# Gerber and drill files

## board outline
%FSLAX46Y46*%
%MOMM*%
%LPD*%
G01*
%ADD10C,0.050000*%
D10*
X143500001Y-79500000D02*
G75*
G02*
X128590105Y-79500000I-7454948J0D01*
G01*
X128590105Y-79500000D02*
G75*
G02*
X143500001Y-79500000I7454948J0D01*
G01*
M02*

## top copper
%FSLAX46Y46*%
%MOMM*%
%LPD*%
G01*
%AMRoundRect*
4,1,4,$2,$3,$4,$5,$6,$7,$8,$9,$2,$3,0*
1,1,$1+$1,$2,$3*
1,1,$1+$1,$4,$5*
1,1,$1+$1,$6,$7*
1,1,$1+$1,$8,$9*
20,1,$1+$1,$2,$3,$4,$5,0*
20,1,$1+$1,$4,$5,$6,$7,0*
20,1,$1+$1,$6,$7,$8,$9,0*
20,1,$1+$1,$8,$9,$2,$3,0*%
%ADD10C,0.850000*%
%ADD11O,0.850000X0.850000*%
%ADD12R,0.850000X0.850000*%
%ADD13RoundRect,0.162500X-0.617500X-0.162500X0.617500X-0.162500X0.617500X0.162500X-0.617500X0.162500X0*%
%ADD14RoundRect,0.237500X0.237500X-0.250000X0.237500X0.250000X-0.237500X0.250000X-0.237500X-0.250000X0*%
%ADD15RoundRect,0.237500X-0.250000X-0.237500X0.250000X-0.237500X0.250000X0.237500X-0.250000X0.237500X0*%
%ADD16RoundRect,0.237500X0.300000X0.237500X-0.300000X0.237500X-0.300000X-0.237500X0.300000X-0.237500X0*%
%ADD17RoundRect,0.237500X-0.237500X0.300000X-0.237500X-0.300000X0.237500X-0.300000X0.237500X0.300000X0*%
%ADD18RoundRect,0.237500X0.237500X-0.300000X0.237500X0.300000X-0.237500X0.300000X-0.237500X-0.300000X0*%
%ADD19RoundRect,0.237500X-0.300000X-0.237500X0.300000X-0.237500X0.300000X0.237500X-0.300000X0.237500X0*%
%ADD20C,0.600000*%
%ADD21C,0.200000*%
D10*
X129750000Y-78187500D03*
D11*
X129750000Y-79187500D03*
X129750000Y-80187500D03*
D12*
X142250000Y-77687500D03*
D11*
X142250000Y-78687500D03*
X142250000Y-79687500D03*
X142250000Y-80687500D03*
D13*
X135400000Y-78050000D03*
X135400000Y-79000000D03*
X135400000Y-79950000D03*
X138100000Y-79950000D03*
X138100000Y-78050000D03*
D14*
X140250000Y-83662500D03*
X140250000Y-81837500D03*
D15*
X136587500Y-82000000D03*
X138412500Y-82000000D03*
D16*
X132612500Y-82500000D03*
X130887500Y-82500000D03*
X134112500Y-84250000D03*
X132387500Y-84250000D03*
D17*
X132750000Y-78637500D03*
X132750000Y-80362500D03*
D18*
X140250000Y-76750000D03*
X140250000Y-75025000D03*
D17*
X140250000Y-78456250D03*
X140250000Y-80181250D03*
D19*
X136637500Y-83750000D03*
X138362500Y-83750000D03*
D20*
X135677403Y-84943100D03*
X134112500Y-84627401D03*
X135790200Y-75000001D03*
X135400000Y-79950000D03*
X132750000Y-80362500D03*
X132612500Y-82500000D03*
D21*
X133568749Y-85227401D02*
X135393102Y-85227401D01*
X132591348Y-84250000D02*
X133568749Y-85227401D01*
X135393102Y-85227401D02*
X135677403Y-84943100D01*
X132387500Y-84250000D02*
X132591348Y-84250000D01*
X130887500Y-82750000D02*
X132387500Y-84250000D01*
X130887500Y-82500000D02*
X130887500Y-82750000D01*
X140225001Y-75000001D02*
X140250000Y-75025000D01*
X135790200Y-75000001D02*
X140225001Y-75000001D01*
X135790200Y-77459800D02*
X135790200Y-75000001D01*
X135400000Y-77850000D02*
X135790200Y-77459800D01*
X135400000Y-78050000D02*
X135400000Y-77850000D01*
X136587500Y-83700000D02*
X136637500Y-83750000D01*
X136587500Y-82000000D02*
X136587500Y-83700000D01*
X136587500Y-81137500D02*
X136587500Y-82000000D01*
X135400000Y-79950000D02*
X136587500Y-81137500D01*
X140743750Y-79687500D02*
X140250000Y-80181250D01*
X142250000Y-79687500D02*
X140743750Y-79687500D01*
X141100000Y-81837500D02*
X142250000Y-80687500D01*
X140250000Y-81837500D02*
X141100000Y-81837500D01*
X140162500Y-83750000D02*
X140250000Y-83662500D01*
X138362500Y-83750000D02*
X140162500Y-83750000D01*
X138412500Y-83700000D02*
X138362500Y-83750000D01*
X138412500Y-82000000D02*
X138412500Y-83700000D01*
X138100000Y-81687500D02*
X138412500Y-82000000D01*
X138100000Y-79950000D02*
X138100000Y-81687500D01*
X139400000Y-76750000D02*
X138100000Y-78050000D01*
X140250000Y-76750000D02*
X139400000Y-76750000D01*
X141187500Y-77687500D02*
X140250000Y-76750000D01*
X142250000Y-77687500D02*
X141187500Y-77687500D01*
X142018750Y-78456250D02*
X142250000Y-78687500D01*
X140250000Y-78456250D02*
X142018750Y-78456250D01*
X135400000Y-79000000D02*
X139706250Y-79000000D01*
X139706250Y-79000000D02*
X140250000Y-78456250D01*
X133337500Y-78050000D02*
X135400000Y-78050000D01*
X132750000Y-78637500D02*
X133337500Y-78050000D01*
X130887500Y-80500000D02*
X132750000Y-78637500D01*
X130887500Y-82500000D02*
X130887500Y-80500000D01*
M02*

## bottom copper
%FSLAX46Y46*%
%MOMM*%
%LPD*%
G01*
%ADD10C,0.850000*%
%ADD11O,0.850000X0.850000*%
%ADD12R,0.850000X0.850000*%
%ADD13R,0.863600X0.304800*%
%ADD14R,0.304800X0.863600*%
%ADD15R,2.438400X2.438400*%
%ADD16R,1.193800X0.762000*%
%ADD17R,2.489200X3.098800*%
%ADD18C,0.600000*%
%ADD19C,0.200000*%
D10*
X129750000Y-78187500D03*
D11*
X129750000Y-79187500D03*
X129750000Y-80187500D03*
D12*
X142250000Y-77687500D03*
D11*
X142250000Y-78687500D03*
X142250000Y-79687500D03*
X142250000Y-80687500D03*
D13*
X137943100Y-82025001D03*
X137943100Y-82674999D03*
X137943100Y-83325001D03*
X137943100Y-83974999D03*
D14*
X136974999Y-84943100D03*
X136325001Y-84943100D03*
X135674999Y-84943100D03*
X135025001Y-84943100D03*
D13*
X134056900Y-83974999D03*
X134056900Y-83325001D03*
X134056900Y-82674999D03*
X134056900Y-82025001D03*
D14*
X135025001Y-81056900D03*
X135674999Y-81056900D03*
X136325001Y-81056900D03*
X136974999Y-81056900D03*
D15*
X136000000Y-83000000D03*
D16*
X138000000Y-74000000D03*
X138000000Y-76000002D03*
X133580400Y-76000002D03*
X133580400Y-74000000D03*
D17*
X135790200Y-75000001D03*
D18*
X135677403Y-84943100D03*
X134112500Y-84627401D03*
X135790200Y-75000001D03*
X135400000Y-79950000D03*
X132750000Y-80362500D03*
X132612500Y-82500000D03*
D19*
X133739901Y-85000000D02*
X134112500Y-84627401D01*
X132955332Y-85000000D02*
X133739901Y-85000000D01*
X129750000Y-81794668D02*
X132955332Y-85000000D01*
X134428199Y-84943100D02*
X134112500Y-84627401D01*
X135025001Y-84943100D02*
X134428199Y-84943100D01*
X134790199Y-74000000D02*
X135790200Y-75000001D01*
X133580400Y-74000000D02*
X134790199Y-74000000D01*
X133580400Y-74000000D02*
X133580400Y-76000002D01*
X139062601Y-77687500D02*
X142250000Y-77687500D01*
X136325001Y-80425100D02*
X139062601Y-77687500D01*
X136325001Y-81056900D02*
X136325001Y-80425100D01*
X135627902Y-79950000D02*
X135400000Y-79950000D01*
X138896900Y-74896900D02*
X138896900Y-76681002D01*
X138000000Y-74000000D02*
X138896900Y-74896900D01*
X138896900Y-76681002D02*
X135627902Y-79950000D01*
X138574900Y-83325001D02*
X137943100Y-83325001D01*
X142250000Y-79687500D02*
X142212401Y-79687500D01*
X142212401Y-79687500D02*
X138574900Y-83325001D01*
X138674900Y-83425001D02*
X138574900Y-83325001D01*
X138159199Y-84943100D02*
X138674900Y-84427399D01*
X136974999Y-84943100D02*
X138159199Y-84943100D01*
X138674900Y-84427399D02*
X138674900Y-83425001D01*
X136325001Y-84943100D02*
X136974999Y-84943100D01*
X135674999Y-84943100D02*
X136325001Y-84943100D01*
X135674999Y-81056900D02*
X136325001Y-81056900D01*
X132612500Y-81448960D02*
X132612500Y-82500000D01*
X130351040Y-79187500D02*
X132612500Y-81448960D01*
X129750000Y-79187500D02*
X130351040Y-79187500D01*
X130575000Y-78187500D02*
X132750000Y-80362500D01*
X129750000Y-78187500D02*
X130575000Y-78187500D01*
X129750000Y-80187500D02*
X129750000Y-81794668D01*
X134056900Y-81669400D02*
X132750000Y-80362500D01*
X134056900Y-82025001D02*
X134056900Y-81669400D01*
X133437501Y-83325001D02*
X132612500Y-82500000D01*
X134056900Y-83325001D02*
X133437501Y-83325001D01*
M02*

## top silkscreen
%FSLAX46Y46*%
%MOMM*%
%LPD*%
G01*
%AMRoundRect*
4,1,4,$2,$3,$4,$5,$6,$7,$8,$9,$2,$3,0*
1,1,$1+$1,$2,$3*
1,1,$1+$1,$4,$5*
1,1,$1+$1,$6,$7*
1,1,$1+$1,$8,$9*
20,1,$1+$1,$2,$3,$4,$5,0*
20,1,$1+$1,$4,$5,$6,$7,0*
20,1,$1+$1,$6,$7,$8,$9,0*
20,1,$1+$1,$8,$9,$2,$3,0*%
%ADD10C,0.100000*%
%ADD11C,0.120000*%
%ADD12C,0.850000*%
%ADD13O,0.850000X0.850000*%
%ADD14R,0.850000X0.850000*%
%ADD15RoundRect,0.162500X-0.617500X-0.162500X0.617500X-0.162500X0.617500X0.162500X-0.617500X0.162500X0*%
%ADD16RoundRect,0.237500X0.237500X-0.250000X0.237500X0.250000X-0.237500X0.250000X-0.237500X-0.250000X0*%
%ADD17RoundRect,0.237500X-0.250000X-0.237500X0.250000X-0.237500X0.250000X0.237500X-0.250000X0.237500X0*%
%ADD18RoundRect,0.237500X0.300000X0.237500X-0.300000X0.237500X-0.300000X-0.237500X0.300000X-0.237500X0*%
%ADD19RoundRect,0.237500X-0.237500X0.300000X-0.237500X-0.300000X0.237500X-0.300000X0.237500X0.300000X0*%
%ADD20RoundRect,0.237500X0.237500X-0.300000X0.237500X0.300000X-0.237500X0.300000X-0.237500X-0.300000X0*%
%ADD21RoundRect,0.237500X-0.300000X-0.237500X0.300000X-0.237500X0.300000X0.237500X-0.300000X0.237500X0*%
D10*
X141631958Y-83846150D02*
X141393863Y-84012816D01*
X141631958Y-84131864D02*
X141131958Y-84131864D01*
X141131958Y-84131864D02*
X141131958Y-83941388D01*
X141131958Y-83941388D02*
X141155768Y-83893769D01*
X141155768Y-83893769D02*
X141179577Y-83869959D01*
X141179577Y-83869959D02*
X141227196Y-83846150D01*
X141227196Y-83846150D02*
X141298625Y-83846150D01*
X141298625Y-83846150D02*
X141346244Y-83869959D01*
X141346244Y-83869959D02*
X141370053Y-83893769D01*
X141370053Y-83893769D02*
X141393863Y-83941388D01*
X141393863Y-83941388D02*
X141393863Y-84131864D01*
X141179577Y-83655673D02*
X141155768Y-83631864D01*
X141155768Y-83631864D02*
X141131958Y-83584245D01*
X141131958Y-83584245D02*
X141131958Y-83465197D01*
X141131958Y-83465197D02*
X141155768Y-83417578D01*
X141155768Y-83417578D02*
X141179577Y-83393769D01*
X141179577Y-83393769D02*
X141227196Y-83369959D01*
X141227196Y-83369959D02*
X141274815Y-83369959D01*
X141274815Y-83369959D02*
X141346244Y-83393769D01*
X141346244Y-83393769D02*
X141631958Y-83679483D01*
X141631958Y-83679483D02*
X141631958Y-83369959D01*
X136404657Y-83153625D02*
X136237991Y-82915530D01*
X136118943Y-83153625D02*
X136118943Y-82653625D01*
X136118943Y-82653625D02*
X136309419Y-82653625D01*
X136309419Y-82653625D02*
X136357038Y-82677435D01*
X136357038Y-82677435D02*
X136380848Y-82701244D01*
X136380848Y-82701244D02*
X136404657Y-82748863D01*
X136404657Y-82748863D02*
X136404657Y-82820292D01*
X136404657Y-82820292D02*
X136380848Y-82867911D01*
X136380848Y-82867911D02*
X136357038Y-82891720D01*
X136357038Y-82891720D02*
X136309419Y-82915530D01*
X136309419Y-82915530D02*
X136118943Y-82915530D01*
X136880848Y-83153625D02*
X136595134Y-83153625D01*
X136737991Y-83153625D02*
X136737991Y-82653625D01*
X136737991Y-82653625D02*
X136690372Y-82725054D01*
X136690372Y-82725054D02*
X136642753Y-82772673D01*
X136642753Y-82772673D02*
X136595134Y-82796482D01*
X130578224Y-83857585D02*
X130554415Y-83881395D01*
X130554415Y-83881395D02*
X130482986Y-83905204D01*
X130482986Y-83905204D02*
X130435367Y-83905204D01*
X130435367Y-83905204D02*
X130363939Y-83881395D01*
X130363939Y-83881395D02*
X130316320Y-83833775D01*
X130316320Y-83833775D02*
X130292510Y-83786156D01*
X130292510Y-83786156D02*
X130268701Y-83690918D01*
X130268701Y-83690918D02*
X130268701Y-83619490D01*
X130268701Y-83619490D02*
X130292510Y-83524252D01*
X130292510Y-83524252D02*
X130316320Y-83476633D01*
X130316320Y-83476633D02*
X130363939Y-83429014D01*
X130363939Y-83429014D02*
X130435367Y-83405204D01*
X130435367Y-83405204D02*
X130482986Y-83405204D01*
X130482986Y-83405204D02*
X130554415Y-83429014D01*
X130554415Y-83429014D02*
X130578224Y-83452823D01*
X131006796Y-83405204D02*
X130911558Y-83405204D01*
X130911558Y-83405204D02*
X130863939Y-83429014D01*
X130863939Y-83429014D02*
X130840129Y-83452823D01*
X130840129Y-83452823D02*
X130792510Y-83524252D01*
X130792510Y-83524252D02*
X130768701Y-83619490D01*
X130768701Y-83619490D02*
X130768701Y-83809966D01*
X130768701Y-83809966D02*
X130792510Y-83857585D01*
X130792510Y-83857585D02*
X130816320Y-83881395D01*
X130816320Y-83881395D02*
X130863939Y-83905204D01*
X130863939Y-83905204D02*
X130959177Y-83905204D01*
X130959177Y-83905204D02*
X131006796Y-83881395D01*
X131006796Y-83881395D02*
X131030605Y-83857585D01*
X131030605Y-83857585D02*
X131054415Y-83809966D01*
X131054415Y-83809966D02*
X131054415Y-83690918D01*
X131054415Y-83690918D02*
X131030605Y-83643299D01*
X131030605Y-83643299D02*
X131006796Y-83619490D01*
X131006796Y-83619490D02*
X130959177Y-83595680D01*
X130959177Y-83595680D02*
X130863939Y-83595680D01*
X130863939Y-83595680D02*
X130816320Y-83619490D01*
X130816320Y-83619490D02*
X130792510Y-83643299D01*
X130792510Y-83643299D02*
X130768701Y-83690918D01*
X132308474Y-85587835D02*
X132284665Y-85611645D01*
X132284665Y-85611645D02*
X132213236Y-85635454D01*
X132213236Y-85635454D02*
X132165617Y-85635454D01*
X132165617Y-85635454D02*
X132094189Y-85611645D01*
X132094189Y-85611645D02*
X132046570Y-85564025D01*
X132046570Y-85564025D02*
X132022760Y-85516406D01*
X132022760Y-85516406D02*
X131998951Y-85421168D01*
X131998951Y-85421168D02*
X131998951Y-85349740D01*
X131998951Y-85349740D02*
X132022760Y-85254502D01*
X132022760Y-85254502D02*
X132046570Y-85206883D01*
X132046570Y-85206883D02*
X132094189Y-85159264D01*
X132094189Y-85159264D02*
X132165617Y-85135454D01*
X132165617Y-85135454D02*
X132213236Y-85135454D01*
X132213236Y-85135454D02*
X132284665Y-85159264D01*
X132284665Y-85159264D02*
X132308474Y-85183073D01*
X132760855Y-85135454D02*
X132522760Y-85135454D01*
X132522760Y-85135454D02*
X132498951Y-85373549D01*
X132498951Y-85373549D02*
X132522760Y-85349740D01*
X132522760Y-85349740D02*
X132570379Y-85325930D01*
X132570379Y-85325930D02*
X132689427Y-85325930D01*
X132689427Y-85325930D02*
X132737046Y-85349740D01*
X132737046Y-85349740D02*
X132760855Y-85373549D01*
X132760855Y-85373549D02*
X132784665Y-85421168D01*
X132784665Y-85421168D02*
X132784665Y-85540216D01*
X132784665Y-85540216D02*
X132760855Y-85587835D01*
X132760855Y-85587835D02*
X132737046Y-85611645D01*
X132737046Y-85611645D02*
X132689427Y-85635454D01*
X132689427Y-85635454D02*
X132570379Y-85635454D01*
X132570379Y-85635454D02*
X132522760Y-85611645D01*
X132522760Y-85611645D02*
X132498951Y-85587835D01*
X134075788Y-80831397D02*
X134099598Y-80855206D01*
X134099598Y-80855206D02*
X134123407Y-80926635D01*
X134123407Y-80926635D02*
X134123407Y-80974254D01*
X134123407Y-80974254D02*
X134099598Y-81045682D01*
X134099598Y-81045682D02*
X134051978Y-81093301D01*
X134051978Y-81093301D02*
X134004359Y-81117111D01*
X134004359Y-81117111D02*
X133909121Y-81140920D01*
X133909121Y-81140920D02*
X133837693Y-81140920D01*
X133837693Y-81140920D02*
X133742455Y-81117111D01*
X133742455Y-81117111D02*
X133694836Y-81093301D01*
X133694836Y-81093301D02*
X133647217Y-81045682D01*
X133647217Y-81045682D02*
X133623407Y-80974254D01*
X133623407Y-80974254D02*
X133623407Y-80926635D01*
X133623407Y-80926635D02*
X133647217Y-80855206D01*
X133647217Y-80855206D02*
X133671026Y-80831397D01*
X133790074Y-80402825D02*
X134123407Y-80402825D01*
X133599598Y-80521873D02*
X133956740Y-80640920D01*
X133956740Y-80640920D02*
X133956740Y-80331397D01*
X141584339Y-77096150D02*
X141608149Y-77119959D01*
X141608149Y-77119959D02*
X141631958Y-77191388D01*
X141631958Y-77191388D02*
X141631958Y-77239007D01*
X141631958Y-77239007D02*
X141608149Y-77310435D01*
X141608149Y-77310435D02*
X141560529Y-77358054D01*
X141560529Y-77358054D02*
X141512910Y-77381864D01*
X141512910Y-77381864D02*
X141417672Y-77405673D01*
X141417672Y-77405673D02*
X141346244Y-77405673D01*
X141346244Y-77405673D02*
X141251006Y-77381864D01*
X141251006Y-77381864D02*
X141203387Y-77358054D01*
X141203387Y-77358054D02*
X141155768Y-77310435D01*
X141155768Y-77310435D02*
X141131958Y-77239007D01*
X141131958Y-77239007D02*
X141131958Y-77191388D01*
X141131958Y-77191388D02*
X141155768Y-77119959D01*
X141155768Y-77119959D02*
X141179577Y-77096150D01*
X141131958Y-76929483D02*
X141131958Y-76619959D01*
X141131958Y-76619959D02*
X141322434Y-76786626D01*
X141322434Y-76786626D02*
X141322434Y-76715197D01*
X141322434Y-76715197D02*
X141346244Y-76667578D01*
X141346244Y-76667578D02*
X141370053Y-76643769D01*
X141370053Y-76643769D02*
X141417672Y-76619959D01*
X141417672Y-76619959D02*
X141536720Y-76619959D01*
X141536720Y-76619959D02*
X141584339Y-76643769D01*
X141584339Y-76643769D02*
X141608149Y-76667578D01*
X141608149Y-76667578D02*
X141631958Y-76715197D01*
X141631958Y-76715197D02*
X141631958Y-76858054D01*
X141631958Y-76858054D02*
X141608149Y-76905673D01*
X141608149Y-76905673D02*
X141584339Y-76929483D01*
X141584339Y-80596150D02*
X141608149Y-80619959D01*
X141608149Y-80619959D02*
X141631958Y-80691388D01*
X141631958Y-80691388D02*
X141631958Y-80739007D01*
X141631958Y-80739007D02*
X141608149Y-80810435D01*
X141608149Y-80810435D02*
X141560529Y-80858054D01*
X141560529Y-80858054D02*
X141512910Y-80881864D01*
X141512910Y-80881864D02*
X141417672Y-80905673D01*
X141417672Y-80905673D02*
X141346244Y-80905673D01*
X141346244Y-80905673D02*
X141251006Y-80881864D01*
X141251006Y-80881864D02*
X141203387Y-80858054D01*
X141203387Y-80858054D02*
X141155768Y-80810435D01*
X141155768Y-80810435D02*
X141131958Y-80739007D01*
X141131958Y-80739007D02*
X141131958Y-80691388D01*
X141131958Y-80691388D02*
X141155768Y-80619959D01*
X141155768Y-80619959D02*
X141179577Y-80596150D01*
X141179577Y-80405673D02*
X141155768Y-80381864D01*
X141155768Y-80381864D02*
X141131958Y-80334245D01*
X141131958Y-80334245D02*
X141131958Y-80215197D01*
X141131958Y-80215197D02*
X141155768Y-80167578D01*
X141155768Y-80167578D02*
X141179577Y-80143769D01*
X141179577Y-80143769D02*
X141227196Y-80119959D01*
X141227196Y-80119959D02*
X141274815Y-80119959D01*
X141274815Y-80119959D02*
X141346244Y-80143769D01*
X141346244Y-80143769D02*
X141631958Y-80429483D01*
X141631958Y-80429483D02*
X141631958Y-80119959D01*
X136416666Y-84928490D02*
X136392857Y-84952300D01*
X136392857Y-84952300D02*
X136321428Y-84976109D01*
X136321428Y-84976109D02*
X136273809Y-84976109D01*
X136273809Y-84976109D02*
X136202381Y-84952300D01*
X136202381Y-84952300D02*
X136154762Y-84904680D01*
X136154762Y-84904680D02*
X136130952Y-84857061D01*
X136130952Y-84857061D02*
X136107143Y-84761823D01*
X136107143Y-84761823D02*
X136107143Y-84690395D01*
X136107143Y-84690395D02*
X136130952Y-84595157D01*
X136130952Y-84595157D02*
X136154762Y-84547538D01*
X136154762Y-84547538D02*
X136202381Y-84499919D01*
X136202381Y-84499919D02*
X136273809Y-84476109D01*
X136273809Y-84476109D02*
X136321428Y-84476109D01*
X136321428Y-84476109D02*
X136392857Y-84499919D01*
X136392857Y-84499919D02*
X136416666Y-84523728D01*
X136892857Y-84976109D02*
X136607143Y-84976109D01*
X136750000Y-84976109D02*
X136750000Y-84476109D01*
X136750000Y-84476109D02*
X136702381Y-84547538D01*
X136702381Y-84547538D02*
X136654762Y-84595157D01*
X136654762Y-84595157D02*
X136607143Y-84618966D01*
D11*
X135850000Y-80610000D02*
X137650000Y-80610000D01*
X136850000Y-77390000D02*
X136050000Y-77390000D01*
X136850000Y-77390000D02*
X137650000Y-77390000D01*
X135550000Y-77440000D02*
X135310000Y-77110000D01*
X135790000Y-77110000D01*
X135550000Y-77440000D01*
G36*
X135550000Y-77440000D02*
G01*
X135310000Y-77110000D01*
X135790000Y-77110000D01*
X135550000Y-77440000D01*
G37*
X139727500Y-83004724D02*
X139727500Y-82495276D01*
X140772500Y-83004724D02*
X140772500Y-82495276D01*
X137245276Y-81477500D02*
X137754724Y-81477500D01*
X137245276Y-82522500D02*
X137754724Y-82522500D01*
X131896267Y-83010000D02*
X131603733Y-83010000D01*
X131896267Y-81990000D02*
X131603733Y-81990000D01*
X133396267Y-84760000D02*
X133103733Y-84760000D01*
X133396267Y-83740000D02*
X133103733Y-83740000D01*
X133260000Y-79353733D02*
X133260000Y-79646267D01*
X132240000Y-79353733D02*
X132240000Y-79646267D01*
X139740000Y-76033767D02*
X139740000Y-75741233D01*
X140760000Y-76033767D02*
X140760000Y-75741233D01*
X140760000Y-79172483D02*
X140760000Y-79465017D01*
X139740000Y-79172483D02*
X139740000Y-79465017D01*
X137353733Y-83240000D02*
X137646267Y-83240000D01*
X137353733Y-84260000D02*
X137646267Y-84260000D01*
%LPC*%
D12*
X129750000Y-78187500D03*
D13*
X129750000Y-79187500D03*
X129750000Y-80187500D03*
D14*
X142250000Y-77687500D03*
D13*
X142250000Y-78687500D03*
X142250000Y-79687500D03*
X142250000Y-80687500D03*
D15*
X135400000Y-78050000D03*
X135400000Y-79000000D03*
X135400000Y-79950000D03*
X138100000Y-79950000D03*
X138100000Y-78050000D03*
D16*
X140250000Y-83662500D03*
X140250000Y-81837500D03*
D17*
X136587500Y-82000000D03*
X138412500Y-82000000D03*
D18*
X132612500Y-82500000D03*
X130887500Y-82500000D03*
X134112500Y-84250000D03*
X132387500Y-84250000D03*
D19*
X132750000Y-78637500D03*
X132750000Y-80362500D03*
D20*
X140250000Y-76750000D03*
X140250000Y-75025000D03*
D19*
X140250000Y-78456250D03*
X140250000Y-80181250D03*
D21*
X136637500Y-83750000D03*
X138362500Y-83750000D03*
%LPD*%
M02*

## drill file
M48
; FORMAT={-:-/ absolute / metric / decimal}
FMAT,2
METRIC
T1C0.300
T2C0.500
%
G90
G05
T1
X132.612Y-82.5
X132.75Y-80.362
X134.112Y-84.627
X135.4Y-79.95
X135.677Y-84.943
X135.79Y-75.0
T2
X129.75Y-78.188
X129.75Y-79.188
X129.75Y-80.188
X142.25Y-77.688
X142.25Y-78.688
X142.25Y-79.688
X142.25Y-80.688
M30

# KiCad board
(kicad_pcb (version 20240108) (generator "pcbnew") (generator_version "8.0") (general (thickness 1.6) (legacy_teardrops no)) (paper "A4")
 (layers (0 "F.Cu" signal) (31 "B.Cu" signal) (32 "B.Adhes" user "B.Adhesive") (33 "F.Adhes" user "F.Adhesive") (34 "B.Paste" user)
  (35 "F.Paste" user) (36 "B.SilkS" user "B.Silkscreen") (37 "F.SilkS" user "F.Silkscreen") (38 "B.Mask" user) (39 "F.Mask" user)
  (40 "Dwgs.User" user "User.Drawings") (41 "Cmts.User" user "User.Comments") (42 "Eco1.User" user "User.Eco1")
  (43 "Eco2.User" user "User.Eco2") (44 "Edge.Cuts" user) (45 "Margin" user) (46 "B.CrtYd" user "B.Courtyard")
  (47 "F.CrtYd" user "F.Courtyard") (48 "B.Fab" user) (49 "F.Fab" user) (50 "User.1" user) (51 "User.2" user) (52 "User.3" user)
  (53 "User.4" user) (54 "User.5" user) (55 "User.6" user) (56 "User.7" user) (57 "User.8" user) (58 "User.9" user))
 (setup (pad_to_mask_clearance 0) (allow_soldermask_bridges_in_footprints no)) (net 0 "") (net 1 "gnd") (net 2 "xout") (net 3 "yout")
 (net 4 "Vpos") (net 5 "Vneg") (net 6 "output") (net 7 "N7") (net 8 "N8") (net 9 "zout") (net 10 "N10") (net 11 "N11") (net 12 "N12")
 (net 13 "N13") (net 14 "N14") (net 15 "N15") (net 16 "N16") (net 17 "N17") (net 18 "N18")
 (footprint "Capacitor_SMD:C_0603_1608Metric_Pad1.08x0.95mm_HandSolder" (layer "F.Cu") (at 132.75 79.5 -90)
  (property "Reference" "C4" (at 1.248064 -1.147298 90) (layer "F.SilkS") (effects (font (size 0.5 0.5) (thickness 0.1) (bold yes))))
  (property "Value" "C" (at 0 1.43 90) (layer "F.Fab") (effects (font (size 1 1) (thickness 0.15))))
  (fp_line (start -0.146267 0.51) (end 0.146267 0.51) (stroke (width 0.12) (type solid)) (layer "F.SilkS"))
  (fp_line (start -0.146267 -0.51) (end 0.146267 -0.51) (stroke (width 0.12) (type solid)) (layer "F.SilkS"))
  (pad "1" smd roundrect (at -0.8625 0 270) (size 1.075 0.95) (layers "F.Cu" "F.Paste" "F.Mask") (roundrect_rratio 0.25) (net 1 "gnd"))
  (pad "2" smd roundrect (at 0.8625 0 270) (size 1.075 0.95) (layers "F.Cu" "F.Paste" "F.Mask") (roundrect_rratio 0.25) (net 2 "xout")))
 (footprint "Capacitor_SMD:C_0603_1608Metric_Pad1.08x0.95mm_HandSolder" (layer "F.Cu") (at 131.75 82.5 180)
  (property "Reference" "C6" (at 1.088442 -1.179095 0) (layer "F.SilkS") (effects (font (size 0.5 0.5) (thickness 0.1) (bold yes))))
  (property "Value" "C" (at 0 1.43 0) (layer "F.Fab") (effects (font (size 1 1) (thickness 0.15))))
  (fp_line (start -0.146267 0.51) (end 0.146267 0.51) (stroke (width 0.12) (type solid)) (layer "F.SilkS"))
  (fp_line (start -0.146267 -0.51) (end 0.146267 -0.51) (stroke (width 0.12) (type solid)) (layer "F.SilkS"))
  (pad "1" smd roundrect (at -0.8625 0 180) (size 1.075 0.95) (layers "F.Cu" "F.Paste" "F.Mask") (roundrect_rratio 0.25) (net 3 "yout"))
  (pad "2" smd roundrect (at 0.8625 0 180) (size 1.075 0.95) (layers "F.Cu" "F.Paste" "F.Mask") (roundrect_rratio 0.25) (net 1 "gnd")))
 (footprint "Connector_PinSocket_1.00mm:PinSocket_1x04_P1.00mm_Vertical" (layer "F.Cu") (at 142.25 77.6875)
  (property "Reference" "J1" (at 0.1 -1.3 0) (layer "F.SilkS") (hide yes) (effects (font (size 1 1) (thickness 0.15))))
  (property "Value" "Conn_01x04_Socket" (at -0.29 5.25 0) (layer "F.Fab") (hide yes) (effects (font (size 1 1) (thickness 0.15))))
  (pad "1" thru_hole rect (at 0 0) (size 0.85 0.85) (drill 0.5) (layers "*.Cu" "*.Mask") (remove_unused_layers no) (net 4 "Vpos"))
  (pad "2" thru_hole oval (at 0 1) (size 0.85 0.85) (drill 0.5) (layers "*.Cu" "*.Mask") (remove_unused_layers no) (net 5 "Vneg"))
  (pad "3" thru_hole oval (at 0 2) (size 0.85 0.85) (drill 0.5) (layers "*.Cu" "*.Mask") (remove_unused_layers no) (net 1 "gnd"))
  (pad "4" thru_hole oval (at 0 3) (size 0.85 0.85) (drill 0.5) (layers "*.Cu" "*.Mask") (remove_unused_layers no) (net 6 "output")))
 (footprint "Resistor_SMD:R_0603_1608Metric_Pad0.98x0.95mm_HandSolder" (layer "F.Cu") (at 137.5 82)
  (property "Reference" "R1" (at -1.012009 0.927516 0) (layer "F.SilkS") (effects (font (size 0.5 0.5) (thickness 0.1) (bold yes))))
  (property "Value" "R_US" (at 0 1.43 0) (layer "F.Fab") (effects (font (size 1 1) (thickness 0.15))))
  (fp_line (start -0.254724 -0.5225) (end 0.254724 -0.5225) (stroke (width 0.12) (type solid)) (layer "F.SilkS"))
  (fp_line (start -0.254724 0.5225) (end 0.254724 0.5225) (stroke (width 0.12) (type solid)) (layer "F.SilkS"))
  (pad "1" smd roundrect (at -0.9125 0) (size 0.975 0.95) (layers "F.Cu" "F.Paste" "F.Mask") (roundrect_rratio 0.25) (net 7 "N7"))
  (pad "2" smd roundrect (at 0.9125 0) (size 0.975 0.95) (layers "F.Cu" "F.Paste" "F.Mask") (roundrect_rratio 0.25) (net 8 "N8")))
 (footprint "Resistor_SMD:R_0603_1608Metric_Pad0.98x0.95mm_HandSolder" (layer "F.Cu") (at 140.25 82.75 90)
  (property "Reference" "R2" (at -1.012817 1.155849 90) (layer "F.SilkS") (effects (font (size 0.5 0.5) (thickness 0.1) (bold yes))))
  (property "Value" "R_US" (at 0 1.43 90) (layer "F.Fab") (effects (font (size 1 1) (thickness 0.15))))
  (fp_line (start -0.254724 -0.5225) (end 0.254724 -0.5225) (stroke (width 0.12) (type solid)) (layer "F.SilkS"))
  (fp_line (start -0.254724 0.5225) (end 0.254724 0.5225) (stroke (width 0.12) (type solid)) (layer "F.SilkS"))
  (pad "1" smd roundrect (at -0.9125 0 90) (size 0.975 0.95) (layers "F.Cu" "F.Paste" "F.Mask") (roundrect_rratio 0.25) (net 8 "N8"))
  (pad "2" smd roundrect (at 0.9125 0 90) (size 0.975 0.95) (layers "F.Cu" "F.Paste" "F.Mask") (roundrect_rratio 0.25) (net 6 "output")))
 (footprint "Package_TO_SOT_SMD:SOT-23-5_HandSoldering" (layer "F.Cu") (at 136.75 79)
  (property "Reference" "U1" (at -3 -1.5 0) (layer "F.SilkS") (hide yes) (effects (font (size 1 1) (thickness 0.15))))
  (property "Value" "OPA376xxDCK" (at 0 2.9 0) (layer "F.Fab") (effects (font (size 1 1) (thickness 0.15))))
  (fp_line (start -0.9 1.61) (end 0.9 1.61) (stroke (width 0.12) (type solid)) (layer "F.SilkS"))
  (fp_line (start 0.1 -1.61) (end -0.7 -1.61) (stroke (width 0.12) (type solid)) (layer "F.SilkS"))
  (fp_line (start 0.1 -1.61) (end 0.9 -1.61) (stroke (width 0.12) (type solid)) (layer "F.SilkS"))
  (fp_poly
   (pts (xy -1.2 -1.56) (xy -1.44 -1.89) (xy -0.96 -1.89) (xy -1.2 -1.56)) (stroke (width 0.12) (type solid)) (fill solid) (layer "F.SilkS"))
  (pad "1" smd roundrect (at -1.35 -0.95) (size 1.56 0.65) (layers "F.Cu" "F.Paste" "F.Mask") (roundrect_rratio 0.25) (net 1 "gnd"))
  (pad "2" smd roundrect (at -1.35 0) (size 1.56 0.65) (layers "F.Cu" "F.Paste" "F.Mask") (roundrect_rratio 0.25) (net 5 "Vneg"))
  (pad "3" smd roundrect (at -1.35 0.95) (size 1.56 0.65) (layers "F.Cu" "F.Paste" "F.Mask") (roundrect_rratio 0.25) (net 7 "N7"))
  (pad "4" smd roundrect (at 1.35 0.95) (size 1.56 0.65) (layers "F.Cu" "F.Paste" "F.Mask") (roundrect_rratio 0.25) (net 8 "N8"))
  (pad "5" smd roundrect (at 1.35 -0.95) (size 1.56 0.65) (layers "F.Cu" "F.Paste" "F.Mask") (roundrect_rratio 0.25) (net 4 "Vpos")))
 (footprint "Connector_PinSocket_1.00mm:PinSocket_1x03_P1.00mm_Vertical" (layer "F.Cu") (at 129.75 78.1875)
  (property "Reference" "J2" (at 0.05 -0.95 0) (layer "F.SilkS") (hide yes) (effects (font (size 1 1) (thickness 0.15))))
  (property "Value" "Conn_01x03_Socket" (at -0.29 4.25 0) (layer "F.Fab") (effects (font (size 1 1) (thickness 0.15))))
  (pad "1" thru_hole circle (at 0 0) (size 0.85 0.85) (drill 0.5) (layers "*.Cu" "*.Mask") (remove_unused_layers no) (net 2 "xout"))
  (pad "2" thru_hole oval (at 0 1) (size 0.85 0.85) (drill 0.5) (layers "*.Cu" "*.Mask") (remove_unused_layers no) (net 3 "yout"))
  (pad "3" thru_hole oval (at 0 2) (size 0.85 0.85) (drill 0.5) (layers "*.Cu" "*.Mask") (remove_unused_layers no) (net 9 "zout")))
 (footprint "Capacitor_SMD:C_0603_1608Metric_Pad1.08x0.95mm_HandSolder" (layer "F.Cu") (at 140.25 79.31875 -90)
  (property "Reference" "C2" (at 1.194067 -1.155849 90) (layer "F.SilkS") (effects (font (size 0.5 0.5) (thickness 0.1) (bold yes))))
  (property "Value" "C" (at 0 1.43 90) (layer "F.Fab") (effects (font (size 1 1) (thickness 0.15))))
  (fp_line (start -0.146267 0.51) (end 0.146267 0.51) (stroke (width 0.12) (type solid)) (layer "F.SilkS"))
  (fp_line (start -0.146267 -0.51) (end 0.146267 -0.51) (stroke (width 0.12) (type solid)) (layer "F.SilkS"))
  (pad "1" smd roundrect (at -0.8625 0 270) (size 1.075 0.95) (layers "F.Cu" "F.Paste" "F.Mask") (roundrect_rratio 0.25) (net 5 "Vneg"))
  (pad "2" smd roundrect (at 0.8625 0 270) (size 1.075 0.95) (layers "F.Cu" "F.Paste" "F.Mask") (roundrect_rratio 0.25) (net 1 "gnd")))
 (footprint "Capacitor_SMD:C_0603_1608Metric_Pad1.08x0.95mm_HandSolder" (layer "F.Cu") (at 140.25 75.8875 90)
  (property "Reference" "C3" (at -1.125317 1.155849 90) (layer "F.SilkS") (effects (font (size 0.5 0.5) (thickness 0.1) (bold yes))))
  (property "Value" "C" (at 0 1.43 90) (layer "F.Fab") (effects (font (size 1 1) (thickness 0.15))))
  (fp_line (start -0.146267 -0.51) (end 0.146267 -0.51) (stroke (width 0.12) (type solid)) (layer "F.SilkS"))
  (fp_line (start -0.146267 0.51) (end 0.146267 0.51) (stroke (width 0.12) (type solid)) (layer "F.SilkS"))
  (pad "1" smd roundrect (at -0.8625 0 90) (size 1.075 0.95) (layers "F.Cu" "F.Paste" "F.Mask") (roundrect_rratio 0.25) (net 4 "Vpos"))
  (pad "2" smd roundrect (at 0.8625 0 90) (size 1.075 0.95) (layers "F.Cu" "F.Paste" "F.Mask") (roundrect_rratio 0.25) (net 1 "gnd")))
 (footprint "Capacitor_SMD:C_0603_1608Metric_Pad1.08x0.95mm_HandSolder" (layer "F.Cu") (at 133.25 84.25 180)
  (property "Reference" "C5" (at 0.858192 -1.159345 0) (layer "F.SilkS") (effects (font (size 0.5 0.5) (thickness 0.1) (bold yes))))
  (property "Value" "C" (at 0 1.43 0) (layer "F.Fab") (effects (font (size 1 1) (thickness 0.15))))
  (fp_line (start -0.146267 0.51) (end 0.146267 0.51) (stroke (width 0.12) (type solid)) (layer "F.SilkS"))
  (fp_line (start -0.146267 -0.51) (end 0.146267 -0.51) (stroke (width 0.12) (type solid)) (layer "F.SilkS"))
  (pad "1" smd roundrect (at -0.8625 0 180) (size 1.075 0.95) (layers "F.Cu" "F.Paste" "F.Mask") (roundrect_rratio 0.25) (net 9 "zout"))
  (pad "2" smd roundrect (at 0.8625 0 180) (size 1.075 0.95) (layers "F.Cu" "F.Paste" "F.Mask") (roundrect_rratio 0.25) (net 1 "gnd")))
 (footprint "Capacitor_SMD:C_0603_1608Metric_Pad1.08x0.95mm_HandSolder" (layer "F.Cu") (at 137.5 83.75)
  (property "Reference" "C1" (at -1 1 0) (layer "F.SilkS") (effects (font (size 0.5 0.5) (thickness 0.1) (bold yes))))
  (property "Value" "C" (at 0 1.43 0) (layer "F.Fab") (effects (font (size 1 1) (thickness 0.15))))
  (fp_line (start -0.146267 -0.51) (end 0.146267 -0.51) (stroke (width 0.12) (type solid)) (layer "F.SilkS"))
  (fp_line (start -0.146267 0.51) (end 0.146267 0.51) (stroke (width 0.12) (type solid)) (layer "F.SilkS"))
  (pad "1" smd roundrect (at -0.8625 0) (size 1.075 0.95) (layers "F.Cu" "F.Paste" "F.Mask") (roundrect_rratio 0.25) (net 7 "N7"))
  (pad "2" smd roundrect (at 0.8625 0) (size 1.075 0.95) (layers "F.Cu" "F.Paste" "F.Mask") (roundrect_rratio 0.25) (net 8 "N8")))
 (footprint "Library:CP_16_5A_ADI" (layer "B.Cu") (at 136 83 180)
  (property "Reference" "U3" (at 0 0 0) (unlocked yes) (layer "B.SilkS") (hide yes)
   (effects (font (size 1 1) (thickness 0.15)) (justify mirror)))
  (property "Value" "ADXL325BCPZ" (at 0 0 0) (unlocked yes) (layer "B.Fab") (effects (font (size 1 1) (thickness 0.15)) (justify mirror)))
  (pad "1" smd rect (at -1.9431 0.974999 90) (size 0.3048 0.8636) (layers "B.Cu" "B.Paste" "B.Mask") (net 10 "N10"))
  (pad "2" smd rect (at -1.9431 0.325001 90) (size 0.3048 0.8636) (layers "B.Cu" "B.Paste" "B.Mask") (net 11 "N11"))
  (pad "3" smd rect (at -1.9431 -0.325001 90) (size 0.3048 0.8636) (layers "B.Cu" "B.Paste" "B.Mask") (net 1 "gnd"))
  (pad "4" smd rect (at -1.9431 -0.974999 90) (size 0.3048 0.8636) (layers "B.Cu" "B.Paste" "B.Mask") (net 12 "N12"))
  (pad "5" smd rect (at -0.974999 -1.9431 180) (size 0.3048 0.8636) (layers "B.Cu" "B.Paste" "B.Mask") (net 1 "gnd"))
  (pad "6" smd rect (at -0.325001 -1.9431 180) (size 0.3048 0.8636) (layers "B.Cu" "B.Paste" "B.Mask") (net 1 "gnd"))
  (pad "7" smd rect (at 0.325001 -1.9431 180) (size 0.3048 0.8636) (layers "B.Cu" "B.Paste" "B.Mask") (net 1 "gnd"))
  (pad "8" smd rect (at 0.974999 -1.9431 180) (size 0.3048 0.8636) (layers "B.Cu" "B.Paste" "B.Mask") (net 9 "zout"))
  (pad "9" smd rect (at 1.9431 -0.974999 90) (size 0.3048 0.8636) (layers "B.Cu" "B.Paste" "B.Mask") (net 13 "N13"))
  (pad "10" smd rect (at 1.9431 -0.325001 90) (size 0.3048 0.8636) (layers "B.Cu" "B.Paste" "B.Mask") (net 3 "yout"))
  (pad "11" smd rect (at 1.9431 0.325001 90) (size 0.3048 0.8636) (layers "B.Cu" "B.Paste" "B.Mask") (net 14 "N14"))
  (pad "12" smd rect (at 1.9431 0.974999 90) (size 0.3048 0.8636) (layers "B.Cu" "B.Paste" "B.Mask") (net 2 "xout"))
  (pad "13" smd rect (at 0.974999 1.9431 180) (size 0.3048 0.8636) (layers "B.Cu" "B.Paste" "B.Mask") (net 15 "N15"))
  (pad "14" smd rect (at 0.325001 1.9431 180) (size 0.3048 0.8636) (layers "B.Cu" "B.Paste" "B.Mask") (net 4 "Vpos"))
  (pad "15" smd rect (at -0.325001 1.9431 180) (size 0.3048 0.8636) (layers "B.Cu" "B.Paste" "B.Mask") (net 4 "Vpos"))
  (pad "16" smd rect (at -0.974999 1.9431 180) (size 0.3048 0.8636) (layers "B.Cu" "B.Paste" "B.Mask") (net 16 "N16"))
  (pad "17" smd rect (at 0 0 180) (size 2.4384 2.4384) (layers "B.Cu" "B.Paste" "B.Mask") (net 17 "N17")))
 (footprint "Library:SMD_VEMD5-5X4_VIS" (layer "B.Cu") (at 135.7902 75.000001 180)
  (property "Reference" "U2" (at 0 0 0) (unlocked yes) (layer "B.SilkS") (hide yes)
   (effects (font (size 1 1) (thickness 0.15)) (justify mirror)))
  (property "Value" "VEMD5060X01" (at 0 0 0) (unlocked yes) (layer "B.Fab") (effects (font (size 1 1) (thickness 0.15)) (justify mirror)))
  (pad "1" smd rect (at -2.2098 1.000001 180) (size 1.1938 0.762) (layers "B.Cu" "B.Paste" "B.Mask") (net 7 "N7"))
  (pad "2" smd rect (at -2.2098 -1.000001 180) (size 1.1938 0.762) (layers "B.Cu" "B.Paste" "B.Mask") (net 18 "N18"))
  (pad "3" smd rect (at 2.2098 -1.000001 180) (size 1.1938 0.762) (layers "B.Cu" "B.Paste" "B.Mask") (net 1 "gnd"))
  (pad "4" smd rect (at 2.2098 1.000001 180) (size 1.1938 0.762) (layers "B.Cu" "B.Paste" "B.Mask") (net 1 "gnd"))
  (pad "5" smd rect (at 0 0 180) (size 2.4892 3.0988) (layers "B.Cu" "B.Paste" "B.Mask") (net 1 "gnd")))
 (gr_circle (center 136.045053 79.5) (end 143.499822 79.448409) (stroke (width 0.05) (type default)) (fill none) (layer "Edge.Cuts"))
 (segment (start 138.4125 82) (end 138.4125 83.7) (width 0.2) (layer "F.Cu") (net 8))
 (segment (start 138.3625 83.75) (end 140.1625 83.75) (width 0.2) (layer "F.Cu") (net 8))
 (segment (start 140.1625 83.75) (end 140.25 83.6625) (width 0.2) (layer "F.Cu") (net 8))
 (segment (start 138.1 79.95) (end 138.1 81.6875) (width 0.2) (layer "F.Cu") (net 8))
 (segment (start 138.1 81.6875) (end 138.4125 82) (width 0.2) (layer "F.Cu") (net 8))
 (segment (start 138.4125 83.7) (end 138.3625 83.75) (width 0.2) (layer "F.Cu") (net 8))
 (segment (start 140.74375 79.6875) (end 140.25 80.18125) (width 0.2) (layer "F.Cu") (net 1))
 (segment (start 135.4 78.05) (end 135.4 77.85) (width 0.2) (layer "F.Cu") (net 1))
 (segment (start 133.568749 85.227401) (end 135.393102 85.227401) (width 0.2) (layer "F.Cu") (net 1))
 (segment (start 130.8875 82.5) (end 130.8875 80.5) (width 0.2) (layer "F.Cu") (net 1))
 (segment (start 132.75 78.6375) (end 133.3375 78.05) (width 0.2) (layer "F.Cu") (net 1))
 (segment (start 135.7902 75.000001) (end 140.225001 75.000001) (width 0.2) (layer "F.Cu") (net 1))
 (segment (start 132.591348 84.25) (end 133.568749 85.227401) (width 0.2) (layer "F.Cu") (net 1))
 (segment (start 142.25 79.6875) (end 140.74375 79.6875) (width 0.2) (layer "F.Cu") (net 1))
 (segment (start 135.7902 77.4598) (end 135.7902 75.000001) (width 0.2) (layer "F.Cu") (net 1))
 (segment (start 140.225001 75.000001) (end 140.25 75.025) (width 0.2) (layer "F.Cu") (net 1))
 (segment (start 132.3875 84.25) (end 132.591348 84.25) (width 0.2) (layer "F.Cu") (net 1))
 (segment (start 130.8875 82.75) (end 132.3875 84.25) (width 0.2) (layer "F.Cu") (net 1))
 (segment (start 130.8875 82.5) (end 130.8875 82.75) (width 0.2) (layer "F.Cu") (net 1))
 (segment (start 135.393102 85.227401) (end 135.677403 84.9431) (width 0.2) (layer "F.Cu") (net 1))
 (segment (start 133.3375 78.05) (end 135.4 78.05) (width 0.2) (layer "F.Cu") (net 1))
 (segment (start 130.8875 80.5) (end 132.75 78.6375) (width 0.2) (layer "F.Cu") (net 1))
 (segment (start 135.4 77.85) (end 135.7902 77.4598) (width 0.2) (layer "F.Cu") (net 1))
 (via (at 135.7902 75.000001) (size 0.6) (drill 0.3) (layers "F.Cu" "B.Cu") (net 1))
 (via (at 135.677403 84.9431) (size 0.6) (drill 0.3) (layers "F.Cu" "B.Cu") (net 1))
 (segment (start 136.325001 84.9431) (end 136.974999 84.9431) (width 0.2) (layer "B.Cu") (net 1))
 (segment (start 138.5749 83.325001) (end 137.9431 83.325001) (width 0.2) (layer "B.Cu") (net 1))
 (segment (start 138.159199 84.9431) (end 138.6749 84.427399) (width 0.2) (layer "B.Cu") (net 1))
 (segment (start 134.790199 74) (end 135.7902 75.000001) (width 0.2) (layer "B.Cu") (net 1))
 (segment (start 133.5804 74) (end 134.790199 74) (width 0.2) (layer "B.Cu") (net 1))
 (segment (start 133.5804 74) (end 133.5804 76.000002) (width 0.2) (layer "B.Cu") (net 1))
 (segment (start 142.212401 79.6875) (end 138.5749 83.325001) (width 0.2) (layer "B.Cu") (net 1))
 (segment (start 135.674999 84.9431) (end 136.325001 84.9431) (width 0.2) (layer "B.Cu") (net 1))
 (segment (start 138.6749 84.427399) (end 138.6749 83.425001) (width 0.2) (layer "B.Cu") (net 1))
 (segment (start 136.974999 84.9431) (end 138.159199 84.9431) (width 0.2) (layer "B.Cu") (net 1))
 (segment (start 142.25 79.6875) (end 142.212401 79.6875) (width 0.2) (layer "B.Cu") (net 1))
 (segment (start 138.6749 83.425001) (end 138.5749 83.325001) (width 0.2) (layer "B.Cu") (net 1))
 (segment (start 140.25 78.45625) (end 142.01875 78.45625) (width 0.2) (layer "F.Cu") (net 5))
 (segment (start 139.70625 79) (end 140.25 78.45625) (width 0.2) (layer "F.Cu") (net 5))
 (segment (start 142.01875 78.45625) (end 142.25 78.6875) (width 0.2) (layer "F.Cu") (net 5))
 (segment (start 135.4 79) (end 139.70625 79) (width 0.2) (layer "F.Cu") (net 5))
 (segment (start 142.25 77.6875) (end 141.1875 77.6875) (width 0.2) (layer "F.Cu") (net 4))
 (segment (start 139.4 76.75) (end 138.1 78.05) (width 0.2) (layer "F.Cu") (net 4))
 (segment (start 141.1875 77.6875) (end 140.25 76.75) (width 0.2) (layer "F.Cu") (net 4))
 (segment (start 140.25 76.75) (end 139.4 76.75) (width 0.2) (layer "F.Cu") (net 4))
 (segment (start 139.062601 77.6875) (end 142.25 77.6875) (width 0.2) (layer "B.Cu") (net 4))
 (segment (start 136.325001 80.4251) (end 139.062601 77.6875) (width 0.2) (layer "B.Cu") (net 4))
 (segment (start 136.325001 81.0569) (end 136.325001 80.4251) (width 0.2) (layer "B.Cu") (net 4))
 (segment (start 135.674999 81.0569) (end 136.325001 81.0569) (width 0.2) (layer "B.Cu") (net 4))
 (segment (start 141.1 81.8375) (end 142.25 80.6875) (width 0.2) (layer "F.Cu") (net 6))
 (segment (start 140.25 81.8375) (end 141.1 81.8375) (width 0.2) (layer "F.Cu") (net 6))
 (segment (start 136.5875 83.7) (end 136.6375 83.75) (width 0.2) (layer "F.Cu") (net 7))
 (segment (start 136.5875 82) (end 136.5875 83.7) (width 0.2) (layer "F.Cu") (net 7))
 (segment (start 136.5875 81.1375) (end 136.5875 82) (width 0.2) (layer "F.Cu") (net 7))
 (segment (start 135.4 79.95) (end 136.5875 81.1375) (width 0.2) (layer "F.Cu") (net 7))
 (via (at 135.4 79.95) (size 0.6) (drill 0.3) (layers "F.Cu" "B.Cu") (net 7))
 (segment (start 138.8969 74.8969) (end 138.8969 76.681002) (width 0.2) (layer "B.Cu") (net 7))
 (segment (start 135.627902 79.95) (end 135.4 79.95) (width 0.2) (layer "B.Cu") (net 7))
 (segment (start 138 74) (end 138.8969 74.8969) (width 0.2) (layer "B.Cu") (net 7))
 (segment (start 138.8969 76.681002) (end 135.627902 79.95) (width 0.2) (layer "B.Cu") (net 7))
 (via (at 132.75 80.3625) (size 0.6) (drill 0.3) (layers "F.Cu" "B.Cu") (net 2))
 (segment (start 134.0569 82.025001) (end 134.0569 81.6694) (width 0.2) (layer "B.Cu") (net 2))
 (segment (start 130.575 78.1875) (end 132.75 80.3625) (width 0.2) (layer "B.Cu") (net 2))
 (segment (start 129.75 78.1875) (end 130.575 78.1875) (width 0.2) (layer "B.Cu") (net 2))
 (segment (start 134.0569 81.6694) (end 132.75 80.3625) (width 0.2) (layer "B.Cu") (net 2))
 (via (at 134.1125 84.627401) (size 0.6) (drill 0.3) (layers "F.Cu" "B.Cu") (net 9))
 (segment (start 132.955332 85) (end 133.739901 85) (width 0.2) (layer "B.Cu") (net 9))
 (segment (start 129.75 80.1875) (end 129.75 81.794668) (width 0.2) (layer "B.Cu") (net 9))
 (segment (start 129.75 81.794668) (end 132.955332 85) (width 0.2) (layer "B.Cu") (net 9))
 (segment (start 133.739901 85) (end 134.1125 84.627401) (width 0.2) (layer "B.Cu") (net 9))
 (segment (start 135.025001 84.9431) (end 134.428199 84.9431) (width 0.2) (layer "B.Cu") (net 9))
 (segment (start 134.428199 84.9431) (end 134.1125 84.627401) (width 0.2) (layer "B.Cu") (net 9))
 (via (at 132.6125 82.5) (size 0.6) (drill 0.3) (layers "F.Cu" "B.Cu") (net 3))
 (segment (start 129.75 79.1875) (end 130.35104 79.1875) (width 0.2) (layer "B.Cu") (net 3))
 (segment (start 134.0569 83.325001) (end 133.437501 83.325001) (width 0.2) (layer "B.Cu") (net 3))
 (segment (start 132.6125 81.44896) (end 132.6125 82.5) (width 0.2) (layer "B.Cu") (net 3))
 (segment (start 133.437501 83.325001) (end 132.6125 82.5) (width 0.2) (layer "B.Cu") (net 3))
 (segment (start 130.35104 79.1875) (end 132.6125 81.44896) (width 0.2) (layer "B.Cu") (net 3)))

